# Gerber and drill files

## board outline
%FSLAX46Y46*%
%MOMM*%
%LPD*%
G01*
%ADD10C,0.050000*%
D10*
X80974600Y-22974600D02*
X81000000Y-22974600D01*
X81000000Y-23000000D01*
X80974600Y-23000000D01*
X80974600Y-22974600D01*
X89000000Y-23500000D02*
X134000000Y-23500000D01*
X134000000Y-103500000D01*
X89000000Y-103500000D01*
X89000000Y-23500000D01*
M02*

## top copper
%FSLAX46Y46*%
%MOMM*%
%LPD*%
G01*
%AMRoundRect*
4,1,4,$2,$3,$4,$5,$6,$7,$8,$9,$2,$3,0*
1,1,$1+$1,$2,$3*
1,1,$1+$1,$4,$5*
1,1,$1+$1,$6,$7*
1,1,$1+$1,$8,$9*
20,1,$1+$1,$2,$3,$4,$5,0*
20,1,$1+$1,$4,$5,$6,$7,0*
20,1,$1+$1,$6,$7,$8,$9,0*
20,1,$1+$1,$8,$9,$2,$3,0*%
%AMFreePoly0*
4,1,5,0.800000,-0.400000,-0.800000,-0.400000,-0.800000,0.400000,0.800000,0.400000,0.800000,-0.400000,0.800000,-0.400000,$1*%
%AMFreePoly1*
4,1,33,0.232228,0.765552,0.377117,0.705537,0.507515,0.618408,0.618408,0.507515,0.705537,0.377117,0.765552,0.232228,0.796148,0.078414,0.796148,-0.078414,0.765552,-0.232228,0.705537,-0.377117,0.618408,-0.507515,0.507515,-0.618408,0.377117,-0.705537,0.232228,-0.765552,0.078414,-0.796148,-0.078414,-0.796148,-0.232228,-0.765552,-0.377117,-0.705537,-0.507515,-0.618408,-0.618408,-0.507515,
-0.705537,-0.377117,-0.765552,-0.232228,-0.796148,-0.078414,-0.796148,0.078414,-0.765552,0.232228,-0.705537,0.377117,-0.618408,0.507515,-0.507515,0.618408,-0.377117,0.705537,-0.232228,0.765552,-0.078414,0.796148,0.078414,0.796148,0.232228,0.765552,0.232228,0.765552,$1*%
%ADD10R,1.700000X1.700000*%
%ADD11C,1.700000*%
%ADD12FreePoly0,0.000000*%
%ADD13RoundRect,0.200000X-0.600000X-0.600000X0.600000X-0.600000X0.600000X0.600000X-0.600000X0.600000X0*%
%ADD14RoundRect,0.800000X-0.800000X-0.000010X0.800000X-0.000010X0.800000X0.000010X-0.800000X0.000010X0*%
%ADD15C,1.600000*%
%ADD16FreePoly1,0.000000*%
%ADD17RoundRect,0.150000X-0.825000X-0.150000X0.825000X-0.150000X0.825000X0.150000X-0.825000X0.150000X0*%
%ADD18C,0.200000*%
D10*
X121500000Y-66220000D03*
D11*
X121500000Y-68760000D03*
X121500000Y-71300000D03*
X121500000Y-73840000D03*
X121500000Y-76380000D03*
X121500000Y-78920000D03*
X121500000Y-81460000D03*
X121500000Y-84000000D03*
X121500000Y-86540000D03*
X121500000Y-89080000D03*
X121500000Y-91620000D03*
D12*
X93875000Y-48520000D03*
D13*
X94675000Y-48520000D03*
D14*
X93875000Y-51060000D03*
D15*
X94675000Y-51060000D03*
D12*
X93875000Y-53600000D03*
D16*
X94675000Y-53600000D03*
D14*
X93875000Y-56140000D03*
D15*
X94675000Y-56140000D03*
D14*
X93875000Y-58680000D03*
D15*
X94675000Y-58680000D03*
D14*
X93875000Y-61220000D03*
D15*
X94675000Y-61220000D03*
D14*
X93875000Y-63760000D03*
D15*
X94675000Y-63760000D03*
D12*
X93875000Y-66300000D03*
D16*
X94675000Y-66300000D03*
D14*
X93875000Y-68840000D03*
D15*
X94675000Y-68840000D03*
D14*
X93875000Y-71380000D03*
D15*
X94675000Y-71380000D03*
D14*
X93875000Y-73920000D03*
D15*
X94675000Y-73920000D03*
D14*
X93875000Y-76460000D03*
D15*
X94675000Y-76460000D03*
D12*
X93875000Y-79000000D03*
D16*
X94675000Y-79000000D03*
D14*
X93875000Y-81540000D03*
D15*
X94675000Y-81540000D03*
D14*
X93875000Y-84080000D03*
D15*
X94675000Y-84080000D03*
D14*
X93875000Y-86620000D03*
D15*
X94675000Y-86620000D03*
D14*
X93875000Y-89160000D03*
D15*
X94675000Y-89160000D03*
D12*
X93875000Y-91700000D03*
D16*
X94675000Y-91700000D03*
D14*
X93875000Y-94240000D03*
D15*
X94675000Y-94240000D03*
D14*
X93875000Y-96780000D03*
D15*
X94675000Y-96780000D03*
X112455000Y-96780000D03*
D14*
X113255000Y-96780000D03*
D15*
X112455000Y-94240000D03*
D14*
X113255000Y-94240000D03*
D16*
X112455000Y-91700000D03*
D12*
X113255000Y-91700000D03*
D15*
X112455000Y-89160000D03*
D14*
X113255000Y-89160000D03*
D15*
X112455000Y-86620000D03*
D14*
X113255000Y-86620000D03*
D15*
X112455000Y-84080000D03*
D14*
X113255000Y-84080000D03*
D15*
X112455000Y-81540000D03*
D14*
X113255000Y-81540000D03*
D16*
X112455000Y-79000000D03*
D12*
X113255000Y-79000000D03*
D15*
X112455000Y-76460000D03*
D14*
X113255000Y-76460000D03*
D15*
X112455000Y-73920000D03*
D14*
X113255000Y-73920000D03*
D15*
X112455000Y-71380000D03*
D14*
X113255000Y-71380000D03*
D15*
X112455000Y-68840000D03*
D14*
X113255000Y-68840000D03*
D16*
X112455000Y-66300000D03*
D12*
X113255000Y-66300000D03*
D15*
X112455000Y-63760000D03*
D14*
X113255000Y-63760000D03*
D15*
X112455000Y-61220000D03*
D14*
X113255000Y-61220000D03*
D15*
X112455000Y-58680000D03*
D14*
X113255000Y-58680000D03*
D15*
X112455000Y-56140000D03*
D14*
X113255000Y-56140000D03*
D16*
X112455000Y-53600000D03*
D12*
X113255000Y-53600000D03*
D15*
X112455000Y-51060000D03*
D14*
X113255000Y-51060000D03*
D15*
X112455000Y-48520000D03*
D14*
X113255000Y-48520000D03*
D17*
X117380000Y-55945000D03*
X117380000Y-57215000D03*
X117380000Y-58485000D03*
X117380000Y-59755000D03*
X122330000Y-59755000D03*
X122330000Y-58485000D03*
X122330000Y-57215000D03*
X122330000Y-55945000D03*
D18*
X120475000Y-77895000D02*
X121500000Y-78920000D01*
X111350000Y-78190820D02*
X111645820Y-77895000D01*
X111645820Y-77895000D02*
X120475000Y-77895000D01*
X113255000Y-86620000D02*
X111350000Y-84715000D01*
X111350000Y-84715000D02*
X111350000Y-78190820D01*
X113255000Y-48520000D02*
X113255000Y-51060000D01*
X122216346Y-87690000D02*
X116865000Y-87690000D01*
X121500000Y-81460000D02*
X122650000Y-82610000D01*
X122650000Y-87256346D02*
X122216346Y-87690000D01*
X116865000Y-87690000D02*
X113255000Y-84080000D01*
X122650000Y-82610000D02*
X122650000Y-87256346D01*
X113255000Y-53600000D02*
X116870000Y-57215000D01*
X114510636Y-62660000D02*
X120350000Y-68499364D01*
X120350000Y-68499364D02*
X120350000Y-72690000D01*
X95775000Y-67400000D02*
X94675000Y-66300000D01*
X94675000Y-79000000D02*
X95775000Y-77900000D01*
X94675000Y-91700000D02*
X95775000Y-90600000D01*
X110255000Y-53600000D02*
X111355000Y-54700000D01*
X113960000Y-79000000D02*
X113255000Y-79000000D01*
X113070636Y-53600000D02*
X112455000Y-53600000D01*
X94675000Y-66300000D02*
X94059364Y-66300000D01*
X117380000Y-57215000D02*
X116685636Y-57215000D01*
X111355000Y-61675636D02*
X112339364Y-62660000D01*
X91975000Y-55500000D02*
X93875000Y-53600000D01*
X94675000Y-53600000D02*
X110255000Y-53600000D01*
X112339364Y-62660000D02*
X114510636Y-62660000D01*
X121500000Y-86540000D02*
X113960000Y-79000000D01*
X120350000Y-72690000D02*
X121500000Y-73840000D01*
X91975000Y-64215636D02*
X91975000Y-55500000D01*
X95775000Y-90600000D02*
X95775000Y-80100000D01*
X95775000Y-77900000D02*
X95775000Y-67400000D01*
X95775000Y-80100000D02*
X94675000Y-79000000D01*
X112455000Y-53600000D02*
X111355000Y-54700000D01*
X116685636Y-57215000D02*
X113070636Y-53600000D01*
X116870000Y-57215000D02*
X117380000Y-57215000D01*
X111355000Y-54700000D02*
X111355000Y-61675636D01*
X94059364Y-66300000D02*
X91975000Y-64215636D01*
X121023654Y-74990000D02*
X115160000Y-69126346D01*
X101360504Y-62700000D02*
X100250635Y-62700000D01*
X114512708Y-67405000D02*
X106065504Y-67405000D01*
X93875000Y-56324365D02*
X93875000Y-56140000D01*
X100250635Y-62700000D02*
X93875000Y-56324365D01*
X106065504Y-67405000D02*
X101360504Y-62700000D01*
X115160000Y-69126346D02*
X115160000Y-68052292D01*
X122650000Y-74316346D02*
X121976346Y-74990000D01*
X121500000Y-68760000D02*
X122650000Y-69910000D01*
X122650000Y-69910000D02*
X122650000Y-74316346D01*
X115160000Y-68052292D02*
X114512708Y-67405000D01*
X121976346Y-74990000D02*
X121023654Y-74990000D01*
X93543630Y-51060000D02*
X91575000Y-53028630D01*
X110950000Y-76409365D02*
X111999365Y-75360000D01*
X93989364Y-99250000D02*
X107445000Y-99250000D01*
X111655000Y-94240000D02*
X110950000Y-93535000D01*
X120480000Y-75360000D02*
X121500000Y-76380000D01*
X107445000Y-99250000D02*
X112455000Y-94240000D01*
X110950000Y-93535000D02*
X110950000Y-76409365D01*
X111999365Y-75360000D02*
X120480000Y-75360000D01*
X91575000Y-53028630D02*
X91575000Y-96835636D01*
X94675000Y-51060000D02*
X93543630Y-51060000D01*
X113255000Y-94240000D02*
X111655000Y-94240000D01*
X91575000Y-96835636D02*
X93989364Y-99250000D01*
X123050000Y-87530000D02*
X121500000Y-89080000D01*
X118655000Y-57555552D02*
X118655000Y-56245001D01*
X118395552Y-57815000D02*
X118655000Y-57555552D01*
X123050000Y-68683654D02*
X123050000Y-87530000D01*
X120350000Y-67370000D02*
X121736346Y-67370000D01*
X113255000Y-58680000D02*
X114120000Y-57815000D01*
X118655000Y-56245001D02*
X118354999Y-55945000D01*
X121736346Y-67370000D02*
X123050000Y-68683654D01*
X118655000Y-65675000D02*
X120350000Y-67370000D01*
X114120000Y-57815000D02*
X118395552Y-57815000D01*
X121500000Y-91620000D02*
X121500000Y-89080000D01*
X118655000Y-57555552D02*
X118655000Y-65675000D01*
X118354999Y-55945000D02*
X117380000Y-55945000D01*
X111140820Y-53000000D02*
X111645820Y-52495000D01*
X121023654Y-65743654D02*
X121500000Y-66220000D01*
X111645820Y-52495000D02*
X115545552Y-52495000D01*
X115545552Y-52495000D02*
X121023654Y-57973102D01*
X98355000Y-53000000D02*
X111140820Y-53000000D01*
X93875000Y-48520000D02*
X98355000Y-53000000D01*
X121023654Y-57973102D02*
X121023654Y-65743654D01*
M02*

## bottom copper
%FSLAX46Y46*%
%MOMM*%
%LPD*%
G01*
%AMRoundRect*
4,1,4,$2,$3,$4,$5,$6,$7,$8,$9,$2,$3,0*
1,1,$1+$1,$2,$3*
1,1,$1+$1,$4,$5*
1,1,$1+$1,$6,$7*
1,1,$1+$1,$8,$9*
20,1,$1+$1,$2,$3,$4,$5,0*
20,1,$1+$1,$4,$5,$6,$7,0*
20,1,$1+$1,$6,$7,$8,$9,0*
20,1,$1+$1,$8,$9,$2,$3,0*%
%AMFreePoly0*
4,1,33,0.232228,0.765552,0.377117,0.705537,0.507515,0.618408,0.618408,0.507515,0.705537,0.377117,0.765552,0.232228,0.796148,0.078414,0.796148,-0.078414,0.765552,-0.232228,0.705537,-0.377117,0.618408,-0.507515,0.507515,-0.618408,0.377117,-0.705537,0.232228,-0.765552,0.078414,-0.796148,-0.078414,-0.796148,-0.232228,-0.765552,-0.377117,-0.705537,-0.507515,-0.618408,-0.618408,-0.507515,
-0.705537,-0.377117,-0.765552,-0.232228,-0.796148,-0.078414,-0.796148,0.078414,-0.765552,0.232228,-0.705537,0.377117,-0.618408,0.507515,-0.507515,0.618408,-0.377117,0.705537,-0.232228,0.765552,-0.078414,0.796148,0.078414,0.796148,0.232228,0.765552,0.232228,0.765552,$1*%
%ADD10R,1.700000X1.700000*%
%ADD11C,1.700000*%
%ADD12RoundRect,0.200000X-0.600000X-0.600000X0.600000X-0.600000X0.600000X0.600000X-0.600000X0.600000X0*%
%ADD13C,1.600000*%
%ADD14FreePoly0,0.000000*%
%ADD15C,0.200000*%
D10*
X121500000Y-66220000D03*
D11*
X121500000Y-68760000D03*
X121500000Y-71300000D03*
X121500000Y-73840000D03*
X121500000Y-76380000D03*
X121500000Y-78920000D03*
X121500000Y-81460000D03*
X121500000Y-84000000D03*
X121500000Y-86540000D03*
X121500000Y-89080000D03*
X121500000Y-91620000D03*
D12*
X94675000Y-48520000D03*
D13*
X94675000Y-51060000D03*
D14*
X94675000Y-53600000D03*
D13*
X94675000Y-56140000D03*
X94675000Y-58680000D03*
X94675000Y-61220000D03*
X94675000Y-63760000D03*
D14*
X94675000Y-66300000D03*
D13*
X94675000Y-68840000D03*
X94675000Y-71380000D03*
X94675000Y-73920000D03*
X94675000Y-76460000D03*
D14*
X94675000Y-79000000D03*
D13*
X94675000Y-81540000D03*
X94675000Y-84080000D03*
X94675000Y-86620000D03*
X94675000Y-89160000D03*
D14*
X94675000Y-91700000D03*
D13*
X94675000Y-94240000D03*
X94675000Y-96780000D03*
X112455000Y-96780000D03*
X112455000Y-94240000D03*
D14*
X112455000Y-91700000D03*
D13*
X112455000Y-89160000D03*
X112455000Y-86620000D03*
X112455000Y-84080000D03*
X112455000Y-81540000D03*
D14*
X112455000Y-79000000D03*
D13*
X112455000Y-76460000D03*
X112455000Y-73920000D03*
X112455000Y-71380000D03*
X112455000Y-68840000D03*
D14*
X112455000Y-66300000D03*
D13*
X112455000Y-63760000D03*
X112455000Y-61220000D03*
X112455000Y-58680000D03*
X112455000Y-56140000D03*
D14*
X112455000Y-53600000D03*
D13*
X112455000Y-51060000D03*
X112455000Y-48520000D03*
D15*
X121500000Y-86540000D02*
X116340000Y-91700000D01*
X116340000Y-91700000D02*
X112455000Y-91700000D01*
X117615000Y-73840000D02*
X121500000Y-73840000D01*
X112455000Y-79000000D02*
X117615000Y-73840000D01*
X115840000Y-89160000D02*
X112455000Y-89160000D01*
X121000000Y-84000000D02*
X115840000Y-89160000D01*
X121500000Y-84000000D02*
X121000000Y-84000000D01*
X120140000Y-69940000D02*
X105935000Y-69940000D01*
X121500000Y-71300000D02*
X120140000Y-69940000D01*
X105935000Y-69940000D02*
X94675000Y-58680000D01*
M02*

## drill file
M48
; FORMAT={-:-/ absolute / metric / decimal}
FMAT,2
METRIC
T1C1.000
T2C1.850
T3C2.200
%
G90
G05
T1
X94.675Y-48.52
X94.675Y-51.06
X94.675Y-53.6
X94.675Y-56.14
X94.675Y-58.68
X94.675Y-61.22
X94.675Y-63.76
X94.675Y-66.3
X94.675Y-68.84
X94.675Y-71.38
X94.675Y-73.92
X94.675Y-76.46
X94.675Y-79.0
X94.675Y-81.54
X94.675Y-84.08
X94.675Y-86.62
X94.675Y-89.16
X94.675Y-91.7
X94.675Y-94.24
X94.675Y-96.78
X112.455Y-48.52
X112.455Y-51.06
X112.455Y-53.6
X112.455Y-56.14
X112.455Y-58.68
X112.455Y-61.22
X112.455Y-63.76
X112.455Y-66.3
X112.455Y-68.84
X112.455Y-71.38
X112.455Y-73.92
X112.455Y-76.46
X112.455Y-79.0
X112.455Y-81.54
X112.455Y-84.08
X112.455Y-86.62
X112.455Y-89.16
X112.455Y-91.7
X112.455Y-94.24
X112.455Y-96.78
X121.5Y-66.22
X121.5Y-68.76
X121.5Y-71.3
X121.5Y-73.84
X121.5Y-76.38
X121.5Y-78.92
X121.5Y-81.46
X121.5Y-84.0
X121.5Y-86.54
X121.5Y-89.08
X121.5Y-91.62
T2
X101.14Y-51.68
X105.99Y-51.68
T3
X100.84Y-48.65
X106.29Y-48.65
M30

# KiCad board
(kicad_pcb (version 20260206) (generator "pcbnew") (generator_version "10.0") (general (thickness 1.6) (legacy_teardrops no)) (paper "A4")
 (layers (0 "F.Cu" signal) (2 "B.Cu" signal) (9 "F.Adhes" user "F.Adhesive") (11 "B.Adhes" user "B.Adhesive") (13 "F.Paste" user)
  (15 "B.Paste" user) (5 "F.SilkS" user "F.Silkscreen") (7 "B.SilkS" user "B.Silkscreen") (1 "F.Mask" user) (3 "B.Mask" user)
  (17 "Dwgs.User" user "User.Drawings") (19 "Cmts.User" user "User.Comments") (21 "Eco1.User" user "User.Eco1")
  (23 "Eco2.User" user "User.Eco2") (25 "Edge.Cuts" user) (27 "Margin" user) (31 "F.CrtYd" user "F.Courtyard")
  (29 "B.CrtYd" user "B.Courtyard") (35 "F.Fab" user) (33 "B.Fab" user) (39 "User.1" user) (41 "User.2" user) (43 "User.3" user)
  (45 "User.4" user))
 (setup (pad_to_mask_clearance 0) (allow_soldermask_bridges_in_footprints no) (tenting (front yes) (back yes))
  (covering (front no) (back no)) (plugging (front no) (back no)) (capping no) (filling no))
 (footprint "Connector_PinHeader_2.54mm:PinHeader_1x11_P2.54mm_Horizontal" (layer "F.Cu") (at 121.5 66.22)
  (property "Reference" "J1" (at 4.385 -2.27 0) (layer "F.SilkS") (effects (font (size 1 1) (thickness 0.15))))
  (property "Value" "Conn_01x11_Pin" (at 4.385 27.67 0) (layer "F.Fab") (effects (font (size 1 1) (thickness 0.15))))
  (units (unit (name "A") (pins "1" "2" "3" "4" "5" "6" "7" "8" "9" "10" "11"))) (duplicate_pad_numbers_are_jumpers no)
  (pad "1" thru_hole rect (at 0 0) (size 1.7 1.7) (drill 1) (layers "*.Cu" "*.Mask") (remove_unused_layers no) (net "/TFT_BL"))
  (pad "2" thru_hole circle (at 0 2.54) (size 1.7 1.7) (drill 1) (layers "*.Cu" "*.Mask") (remove_unused_layers no) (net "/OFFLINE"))
  (pad "3" thru_hole circle (at 0 5.08) (size 1.7 1.7) (drill 1) (layers "*.Cu" "*.Mask") (remove_unused_layers no) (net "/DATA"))
  (pad "4" thru_hole circle (at 0 7.62) (size 1.7 1.7) (drill 1) (layers "*.Cu" "*.Mask") (remove_unused_layers no) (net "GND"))
  (pad "5" thru_hole circle (at 0 10.16) (size 1.7 1.7) (drill 1) (layers "*.Cu" "*.Mask") (remove_unused_layers no) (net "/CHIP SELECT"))
  (pad "6" thru_hole circle (at 0 12.7) (size 1.7 1.7) (drill 1) (layers "*.Cu" "*.Mask") (remove_unused_layers no) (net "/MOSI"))
  (pad "7" thru_hole circle (at 0 15.24) (size 1.7 1.7) (drill 1) (layers "*.Cu" "*.Mask") (remove_unused_layers no) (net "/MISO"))
  (pad "8" thru_hole circle (at 0 17.78) (size 1.7 1.7) (drill 1) (layers "*.Cu" "*.Mask") (remove_unused_layers no) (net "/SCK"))
  (pad "9" thru_hole circle (at 0 20.32) (size 1.7 1.7) (drill 1) (layers "*.Cu" "*.Mask") (remove_unused_layers no) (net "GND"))
  (pad "10" thru_hole circle (at 0 22.86) (size 1.7 1.7) (drill 1) (layers "*.Cu" "*.Mask") (remove_unused_layers no) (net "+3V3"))
  (pad "11" thru_hole circle (at 0 25.4) (size 1.7 1.7) (drill 1) (layers "*.Cu" "*.Mask") (remove_unused_layers no) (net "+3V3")))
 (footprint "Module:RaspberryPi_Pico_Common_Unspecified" (layer "F.Cu") (at 103.565 72.65)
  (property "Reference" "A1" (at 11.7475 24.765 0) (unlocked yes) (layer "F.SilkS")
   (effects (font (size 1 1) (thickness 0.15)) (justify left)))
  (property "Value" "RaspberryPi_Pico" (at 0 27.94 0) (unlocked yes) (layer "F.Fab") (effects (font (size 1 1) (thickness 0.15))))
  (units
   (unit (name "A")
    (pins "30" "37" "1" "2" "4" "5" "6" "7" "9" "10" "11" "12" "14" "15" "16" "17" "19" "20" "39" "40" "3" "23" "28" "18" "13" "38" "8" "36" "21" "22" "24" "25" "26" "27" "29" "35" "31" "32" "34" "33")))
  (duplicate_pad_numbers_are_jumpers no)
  (pad "" np_thru_hole circle (at -2.725 -24) (size 2.2 2.2) (drill 2.2) (layers "*.Mask"))
  (pad "" np_thru_hole circle (at -2.425 -20.97) (size 1.85 1.85) (drill 1.85) (layers "*.Mask"))
  (pad "" np_thru_hole circle (at 2.425 -20.97) (size 1.85 1.85) (drill 1.85) (layers "*.Mask"))
  (pad "" np_thru_hole circle (at 2.725 -24) (size 2.2 2.2) (drill 2.2) (layers "*.Mask"))
  (pad "1" smd custom (at -9.69 -24.13) (size 1.6 0.8) (layers "F.Cu" "F.Mask") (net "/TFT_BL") (options (clearance outline) (anchor rect))
   (primitives))
  (pad "1" thru_hole roundrect (at -8.89 -24.13) (size 1.6 1.6) (drill 1) (layers "*.Cu" "*.Mask") (remove_unused_layers no)
   (roundrect_rratio 0.125) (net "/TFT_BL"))
  (pad "2" smd roundrect (at -9.69 -21.59) (size 3.2 1.6) (layers "F.Cu" "F.Mask") (roundrect_rratio 0.5) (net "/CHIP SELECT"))
  (pad "2" thru_hole circle (at -8.89 -21.59) (size 1.6 1.6) (drill 1) (layers "*.Cu" "*.Mask") (remove_unused_layers no)
   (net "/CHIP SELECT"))
  (pad "3" smd custom (at -9.69 -19.05) (size 1.6 0.8) (layers "F.Cu" "F.Mask") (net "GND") (options (clearance outline) (anchor rect))
   (primitives))
  (pad "3" thru_hole custom (at -8.89 -19.05) (size 1.6 1.6) (drill 1) (layers "*.Cu" "*.Mask") (remove_unused_layers no) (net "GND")
   (options (clearance outline) (anchor circle)) (primitives))
  (pad "4" smd roundrect (at -9.69 -16.51) (size 3.2 1.6) (layers "F.Cu" "F.Mask") (roundrect_rratio 0.5) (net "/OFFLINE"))
  (pad "4" thru_hole circle (at -8.89 -16.51) (size 1.6 1.6) (drill 1) (layers "*.Cu" "*.Mask") (remove_unused_layers no) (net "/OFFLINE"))
  (pad "5" smd roundrect (at -9.69 -13.97) (size 3.2 1.6) (layers "F.Cu" "F.Mask") (roundrect_rratio 0.5) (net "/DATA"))
  (pad "5" thru_hole circle (at -8.89 -13.97) (size 1.6 1.6) (drill 1) (layers "*.Cu" "*.Mask") (remove_unused_layers no) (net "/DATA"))
  (pad "6" smd roundrect (at -9.69 -11.43) (size 3.2 1.6) (layers "F.Cu" "F.Mask") (roundrect_rratio 0.5)
   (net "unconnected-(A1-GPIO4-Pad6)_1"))
  (pad "6" thru_hole circle (at -8.89 -11.43) (size 1.6 1.6) (drill 1) (layers "*.Cu" "*.Mask") (remove_unused_layers no)
   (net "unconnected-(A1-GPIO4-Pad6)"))
  (pad "7" smd roundrect (at -9.69 -8.89) (size 3.2 1.6) (layers "F.Cu" "F.Mask") (roundrect_rratio 0.5)
   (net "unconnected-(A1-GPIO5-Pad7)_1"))
  (pad "7" thru_hole circle (at -8.89 -8.89) (size 1.6 1.6) (drill 1) (layers "*.Cu" "*.Mask") (remove_unused_layers no)
   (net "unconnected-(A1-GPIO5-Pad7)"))
  (pad "8" smd custom (at -9.69 -6.35) (size 1.6 0.8) (layers "F.Cu" "F.Mask") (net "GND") (options (clearance outline) (anchor rect))
   (primitives))
  (pad "8" thru_hole custom (at -8.89 -6.35) (size 1.6 1.6) (drill 1) (layers "*.Cu" "*.Mask") (remove_unused_layers no) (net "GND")
   (options (clearance outline) (anchor circle)) (primitives))
  (pad "9" smd roundrect (at -9.69 -3.81) (size 3.2 1.6) (layers "F.Cu" "F.Mask") (roundrect_rratio 0.5) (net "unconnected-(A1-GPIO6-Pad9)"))
  (pad "9" thru_hole circle (at -8.89 -3.81) (size 1.6 1.6) (drill 1) (layers "*.Cu" "*.Mask") (remove_unused_layers no)
   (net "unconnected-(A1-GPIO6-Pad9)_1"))
  (pad "10" smd roundrect (at -9.69 -1.27) (size 3.2 1.6) (layers "F.Cu" "F.Mask") (roundrect_rratio 0.5)
   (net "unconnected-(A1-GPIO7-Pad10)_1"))
  (pad "10" thru_hole circle (at -8.89 -1.27) (size 1.6 1.6) (drill 1) (layers "*.Cu" "*.Mask") (remove_unused_layers no)
   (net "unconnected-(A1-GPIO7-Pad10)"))
  (pad "11" smd roundrect (at -9.69 1.27) (size 3.2 1.6) (layers "F.Cu" "F.Mask") (roundrect_rratio 0.5)
   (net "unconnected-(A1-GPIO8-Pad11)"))
  (pad "11" thru_hole circle (at -8.89 1.27) (size 1.6 1.6) (drill 1) (layers "*.Cu" "*.Mask") (remove_unused_layers no)
   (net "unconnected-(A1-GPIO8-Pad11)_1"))
  (pad "12" smd roundrect (at -9.69 3.81) (size 3.2 1.6) (layers "F.Cu" "F.Mask") (roundrect_rratio 0.5)
   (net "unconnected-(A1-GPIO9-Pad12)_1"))
  (pad "12" thru_hole circle (at -8.89 3.81) (size 1.6 1.6) (drill 1) (layers "*.Cu" "*.Mask") (remove_unused_layers no)
   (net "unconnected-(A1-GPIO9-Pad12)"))
  (pad "13" smd custom (at -9.69 6.35) (size 1.6 0.8) (layers "F.Cu" "F.Mask") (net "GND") (options (clearance outline) (anchor rect))
   (primitives))
  (pad "13" thru_hole custom (at -8.89 6.35) (size 1.6 1.6) (drill 1) (layers "*.Cu" "*.Mask") (remove_unused_layers no) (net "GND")
   (options (clearance outline) (anchor circle)) (primitives))
  (pad "14" smd roundrect (at -9.69 8.89) (size 3.2 1.6) (layers "F.Cu" "F.Mask") (roundrect_rratio 0.5)
   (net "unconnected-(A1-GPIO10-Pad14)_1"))
  (pad "14" thru_hole circle (at -8.89 8.89) (size 1.6 1.6) (drill 1) (layers "*.Cu" "*.Mask") (remove_unused_layers no)
   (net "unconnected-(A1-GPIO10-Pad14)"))
  (pad "15" smd roundrect (at -9.69 11.43) (size 3.2 1.6) (layers "F.Cu" "F.Mask") (roundrect_rratio 0.5)
   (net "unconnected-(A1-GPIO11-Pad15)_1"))
  (pad "15" thru_hole circle (at -8.89 11.43) (size 1.6 1.6) (drill 1) (layers "*.Cu" "*.Mask") (remove_unused_layers no)
   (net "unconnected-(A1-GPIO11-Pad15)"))
  (pad "16" smd roundrect (at -9.69 13.97) (size 3.2 1.6) (layers "F.Cu" "F.Mask") (roundrect_rratio 0.5)
   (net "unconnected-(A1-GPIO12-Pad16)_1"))
  (pad "16" thru_hole circle (at -8.89 13.97) (size 1.6 1.6) (drill 1) (layers "*.Cu" "*.Mask") (remove_unused_layers no)
   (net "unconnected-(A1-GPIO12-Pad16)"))
  (pad "17" smd roundrect (at -9.69 16.51) (size 3.2 1.6) (layers "F.Cu" "F.Mask") (roundrect_rratio 0.5)
   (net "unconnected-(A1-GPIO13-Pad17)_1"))
  (pad "17" thru_hole circle (at -8.89 16.51) (size 1.6 1.6) (drill 1) (layers "*.Cu" "*.Mask") (remove_unused_layers no)
   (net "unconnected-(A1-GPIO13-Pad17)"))
  (pad "18" smd custom (at -9.69 19.05) (size 1.6 0.8) (layers "F.Cu" "F.Mask") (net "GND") (options (clearance outline) (anchor rect))
   (primitives))
  (pad "18" thru_hole custom (at -8.89 19.05) (size 1.6 1.6) (drill 1) (layers "*.Cu" "*.Mask") (remove_unused_layers no) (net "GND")
   (options (clearance outline) (anchor circle)) (primitives))
  (pad "19" smd roundrect (at -9.69 21.59) (size 3.2 1.6) (layers "F.Cu" "F.Mask") (roundrect_rratio 0.5)
   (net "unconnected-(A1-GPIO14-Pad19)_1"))
  (pad "19" thru_hole circle (at -8.89 21.59) (size 1.6 1.6) (drill 1) (layers "*.Cu" "*.Mask") (remove_unused_layers no)
   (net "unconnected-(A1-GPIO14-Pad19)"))
  (pad "20" smd roundrect (at -9.69 24.13) (size 3.2 1.6) (layers "F.Cu" "F.Mask") (roundrect_rratio 0.5)
   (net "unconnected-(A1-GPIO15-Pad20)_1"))
  (pad "20" thru_hole circle (at -8.89 24.13) (size 1.6 1.6) (drill 1) (layers "*.Cu" "*.Mask") (remove_unused_layers no)
   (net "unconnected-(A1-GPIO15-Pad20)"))
  (pad "21" thru_hole circle (at 8.89 24.13) (size 1.6 1.6) (drill 1) (layers "*.Cu" "*.Mask") (remove_unused_layers no)
   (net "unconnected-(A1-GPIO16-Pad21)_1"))
  (pad "21" smd roundrect (at 9.69 24.13) (size 3.2 1.6) (layers "F.Cu" "F.Mask") (roundrect_rratio 0.5)
   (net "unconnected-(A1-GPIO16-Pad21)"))
  (pad "22" thru_hole circle (at 8.89 21.59) (size 1.6 1.6) (drill 1) (layers "*.Cu" "*.Mask") (remove_unused_layers no)
   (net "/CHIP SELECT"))
  (pad "22" smd roundrect (at 9.69 21.59) (size 3.2 1.6) (layers "F.Cu" "F.Mask") (roundrect_rratio 0.5) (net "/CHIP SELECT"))
  (pad "23" thru_hole custom (at 8.89 19.05) (size 1.6 1.6) (drill 1) (layers "*.Cu" "*.Mask") (remove_unused_layers no) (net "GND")
   (options (clearance outline) (anchor circle)) (primitives))
  (pad "23" smd custom (at 9.69 19.05) (size 1.6 0.8) (layers "F.Cu" "F.Mask") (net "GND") (options (clearance outline) (anchor rect))
   (primitives))
  (pad "24" thru_hole circle (at 8.89 16.51) (size 1.6 1.6) (drill 1) (layers "*.Cu" "*.Mask") (remove_unused_layers no) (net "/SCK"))
  (pad "24" smd roundrect (at 9.69 16.51) (size 3.2 1.6) (layers "F.Cu" "F.Mask") (roundrect_rratio 0.5) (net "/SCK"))
  (pad "25" thru_hole circle (at 8.89 13.97) (size 1.6 1.6) (drill 1) (layers "*.Cu" "*.Mask") (remove_unused_layers no) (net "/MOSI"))
  (pad "25" smd roundrect (at 9.69 13.97) (size 3.2 1.6) (layers "F.Cu" "F.Mask") (roundrect_rratio 0.5) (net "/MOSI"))
  (pad "26" thru_hole circle (at 8.89 11.43) (size 1.6 1.6) (drill 1) (layers "*.Cu" "*.Mask") (remove_unused_layers no) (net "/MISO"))
  (pad "26" smd roundrect (at 9.69 11.43) (size 3.2 1.6) (layers "F.Cu" "F.Mask") (roundrect_rratio 0.5) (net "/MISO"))
  (pad "27" thru_hole circle (at 8.89 8.89) (size 1.6 1.6) (drill 1) (layers "*.Cu" "*.Mask") (remove_unused_layers no)
   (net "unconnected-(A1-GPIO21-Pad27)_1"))
  (pad "27" smd roundrect (at 9.69 8.89) (size 3.2 1.6) (layers "F.Cu" "F.Mask") (roundrect_rratio 0.5)
   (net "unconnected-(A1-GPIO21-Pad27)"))
  (pad "28" thru_hole custom (at 8.89 6.35) (size 1.6 1.6) (drill 1) (layers "*.Cu" "*.Mask") (remove_unused_layers no) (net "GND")
   (options (clearance outline) (anchor circle)) (primitives))
  (pad "28" smd custom (at 9.69 6.35) (size 1.6 0.8) (layers "F.Cu" "F.Mask") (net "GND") (options (clearance outline) (anchor rect))
   (primitives))
  (pad "29" thru_hole circle (at 8.89 3.81) (size 1.6 1.6) (drill 1) (layers "*.Cu" "*.Mask") (remove_unused_layers no)
   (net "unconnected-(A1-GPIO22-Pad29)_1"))
  (pad "29" smd roundrect (at 9.69 3.81) (size 3.2 1.6) (layers "F.Cu" "F.Mask") (roundrect_rratio 0.5)
   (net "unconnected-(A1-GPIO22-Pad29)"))
  (pad "30" thru_hole circle (at 8.89 1.27) (size 1.6 1.6) (drill 1) (layers "*.Cu" "*.Mask") (remove_unused_layers no)
   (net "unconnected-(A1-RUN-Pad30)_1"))
  (pad "30" smd roundrect (at 9.69 1.27) (size 3.2 1.6) (layers "F.Cu" "F.Mask") (roundrect_rratio 0.5) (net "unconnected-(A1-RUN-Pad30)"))
  (pad "31" thru_hole circle (at 8.89 -1.27) (size 1.6 1.6) (drill 1) (layers "*.Cu" "*.Mask") (remove_unused_layers no)
   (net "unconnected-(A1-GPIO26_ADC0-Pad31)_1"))
  (pad "31" smd roundrect (at 9.69 -1.27) (size 3.2 1.6) (layers "F.Cu" "F.Mask") (roundrect_rratio 0.5)
   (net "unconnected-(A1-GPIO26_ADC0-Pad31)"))
  (pad "32" thru_hole circle (at 8.89 -3.81) (size 1.6 1.6) (drill 1) (layers "*.Cu" "*.Mask") (remove_unused_layers no)
   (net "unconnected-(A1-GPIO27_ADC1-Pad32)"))
  (pad "32" smd roundrect (at 9.69 -3.81) (size 3.2 1.6) (layers "F.Cu" "F.Mask") (roundrect_rratio 0.5)
   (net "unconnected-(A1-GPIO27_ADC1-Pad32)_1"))
  (pad "33" thru_hole custom (at 8.89 -6.35) (size 1.6 1.6) (drill 1) (layers "*.Cu" "*.Mask") (remove_unused_layers no) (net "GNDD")
   (options (clearance outline) (anchor circle)) (primitives))
  (pad "33" smd custom (at 9.69 -6.35) (size 1.6 0.8) (layers "F.Cu" "F.Mask") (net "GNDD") (options (clearance outline) (anchor rect))
   (primitives))
  (pad "34" thru_hole circle (at 8.89 -8.89) (size 1.6 1.6) (drill 1) (layers "*.Cu" "*.Mask") (remove_unused_layers no)
   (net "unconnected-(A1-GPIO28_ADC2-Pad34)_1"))
  (pad "34" smd roundrect (at 9.69 -8.89) (size 3.2 1.6) (layers "F.Cu" "F.Mask") (roundrect_rratio 0.5)
   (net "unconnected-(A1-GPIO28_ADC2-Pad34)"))
  (pad "35" thru_hole circle (at 8.89 -11.43) (size 1.6 1.6) (drill 1) (layers "*.Cu" "*.Mask") (remove_unused_layers no)
   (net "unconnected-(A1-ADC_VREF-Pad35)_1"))
  (pad "35" smd roundrect (at 9.69 -11.43) (size 3.2 1.6) (layers "F.Cu" "F.Mask") (roundrect_rratio 0.5)
   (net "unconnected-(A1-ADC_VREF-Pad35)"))
  (pad "36" thru_hole circle (at 8.89 -13.97) (size 1.6 1.6) (drill 1) (layers "*.Cu" "*.Mask") (remove_unused_layers no) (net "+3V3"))
  (pad "36" smd roundrect (at 9.69 -13.97) (size 3.2 1.6) (layers "F.Cu" "F.Mask") (roundrect_rratio 0.5) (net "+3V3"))
  (pad "37" thru_hole circle (at 8.89 -16.51) (size 1.6 1.6) (drill 1) (layers "*.Cu" "*.Mask") (remove_unused_layers no)
   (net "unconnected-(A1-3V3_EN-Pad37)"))
  (pad "37" smd roundrect (at 9.69 -16.51) (size 3.2 1.6) (layers "F.Cu" "F.Mask") (roundrect_rratio 0.5)
   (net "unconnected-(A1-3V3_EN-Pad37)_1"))
  (pad "38" thru_hole custom (at 8.89 -19.05) (size 1.6 1.6) (drill 1) (layers "*.Cu" "*.Mask") (remove_unused_layers no) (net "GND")
   (options (clearance outline) (anchor circle)) (primitives))
  (pad "38" smd custom (at 9.69 -19.05) (size 1.6 0.8) (layers "F.Cu" "F.Mask") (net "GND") (options (clearance outline) (anchor rect))
   (primitives))
  (pad "39" thru_hole circle (at 8.89 -21.59) (size 1.6 1.6) (drill 1) (layers "*.Cu" "*.Mask") (remove_unused_layers no) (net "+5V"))
  (pad "39" smd roundrect (at 9.69 -21.59) (size 3.2 1.6) (layers "F.Cu" "F.Mask") (roundrect_rratio 0.5) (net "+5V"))
  (pad "40" thru_hole circle (at 8.89 -24.13) (size 1.6 1.6) (drill 1) (layers "*.Cu" "*.Mask") (remove_unused_layers no) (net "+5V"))
  (pad "40" smd roundrect (at 9.69 -24.13) (size 3.2 1.6) (layers "F.Cu" "F.Mask") (roundrect_rratio 0.5) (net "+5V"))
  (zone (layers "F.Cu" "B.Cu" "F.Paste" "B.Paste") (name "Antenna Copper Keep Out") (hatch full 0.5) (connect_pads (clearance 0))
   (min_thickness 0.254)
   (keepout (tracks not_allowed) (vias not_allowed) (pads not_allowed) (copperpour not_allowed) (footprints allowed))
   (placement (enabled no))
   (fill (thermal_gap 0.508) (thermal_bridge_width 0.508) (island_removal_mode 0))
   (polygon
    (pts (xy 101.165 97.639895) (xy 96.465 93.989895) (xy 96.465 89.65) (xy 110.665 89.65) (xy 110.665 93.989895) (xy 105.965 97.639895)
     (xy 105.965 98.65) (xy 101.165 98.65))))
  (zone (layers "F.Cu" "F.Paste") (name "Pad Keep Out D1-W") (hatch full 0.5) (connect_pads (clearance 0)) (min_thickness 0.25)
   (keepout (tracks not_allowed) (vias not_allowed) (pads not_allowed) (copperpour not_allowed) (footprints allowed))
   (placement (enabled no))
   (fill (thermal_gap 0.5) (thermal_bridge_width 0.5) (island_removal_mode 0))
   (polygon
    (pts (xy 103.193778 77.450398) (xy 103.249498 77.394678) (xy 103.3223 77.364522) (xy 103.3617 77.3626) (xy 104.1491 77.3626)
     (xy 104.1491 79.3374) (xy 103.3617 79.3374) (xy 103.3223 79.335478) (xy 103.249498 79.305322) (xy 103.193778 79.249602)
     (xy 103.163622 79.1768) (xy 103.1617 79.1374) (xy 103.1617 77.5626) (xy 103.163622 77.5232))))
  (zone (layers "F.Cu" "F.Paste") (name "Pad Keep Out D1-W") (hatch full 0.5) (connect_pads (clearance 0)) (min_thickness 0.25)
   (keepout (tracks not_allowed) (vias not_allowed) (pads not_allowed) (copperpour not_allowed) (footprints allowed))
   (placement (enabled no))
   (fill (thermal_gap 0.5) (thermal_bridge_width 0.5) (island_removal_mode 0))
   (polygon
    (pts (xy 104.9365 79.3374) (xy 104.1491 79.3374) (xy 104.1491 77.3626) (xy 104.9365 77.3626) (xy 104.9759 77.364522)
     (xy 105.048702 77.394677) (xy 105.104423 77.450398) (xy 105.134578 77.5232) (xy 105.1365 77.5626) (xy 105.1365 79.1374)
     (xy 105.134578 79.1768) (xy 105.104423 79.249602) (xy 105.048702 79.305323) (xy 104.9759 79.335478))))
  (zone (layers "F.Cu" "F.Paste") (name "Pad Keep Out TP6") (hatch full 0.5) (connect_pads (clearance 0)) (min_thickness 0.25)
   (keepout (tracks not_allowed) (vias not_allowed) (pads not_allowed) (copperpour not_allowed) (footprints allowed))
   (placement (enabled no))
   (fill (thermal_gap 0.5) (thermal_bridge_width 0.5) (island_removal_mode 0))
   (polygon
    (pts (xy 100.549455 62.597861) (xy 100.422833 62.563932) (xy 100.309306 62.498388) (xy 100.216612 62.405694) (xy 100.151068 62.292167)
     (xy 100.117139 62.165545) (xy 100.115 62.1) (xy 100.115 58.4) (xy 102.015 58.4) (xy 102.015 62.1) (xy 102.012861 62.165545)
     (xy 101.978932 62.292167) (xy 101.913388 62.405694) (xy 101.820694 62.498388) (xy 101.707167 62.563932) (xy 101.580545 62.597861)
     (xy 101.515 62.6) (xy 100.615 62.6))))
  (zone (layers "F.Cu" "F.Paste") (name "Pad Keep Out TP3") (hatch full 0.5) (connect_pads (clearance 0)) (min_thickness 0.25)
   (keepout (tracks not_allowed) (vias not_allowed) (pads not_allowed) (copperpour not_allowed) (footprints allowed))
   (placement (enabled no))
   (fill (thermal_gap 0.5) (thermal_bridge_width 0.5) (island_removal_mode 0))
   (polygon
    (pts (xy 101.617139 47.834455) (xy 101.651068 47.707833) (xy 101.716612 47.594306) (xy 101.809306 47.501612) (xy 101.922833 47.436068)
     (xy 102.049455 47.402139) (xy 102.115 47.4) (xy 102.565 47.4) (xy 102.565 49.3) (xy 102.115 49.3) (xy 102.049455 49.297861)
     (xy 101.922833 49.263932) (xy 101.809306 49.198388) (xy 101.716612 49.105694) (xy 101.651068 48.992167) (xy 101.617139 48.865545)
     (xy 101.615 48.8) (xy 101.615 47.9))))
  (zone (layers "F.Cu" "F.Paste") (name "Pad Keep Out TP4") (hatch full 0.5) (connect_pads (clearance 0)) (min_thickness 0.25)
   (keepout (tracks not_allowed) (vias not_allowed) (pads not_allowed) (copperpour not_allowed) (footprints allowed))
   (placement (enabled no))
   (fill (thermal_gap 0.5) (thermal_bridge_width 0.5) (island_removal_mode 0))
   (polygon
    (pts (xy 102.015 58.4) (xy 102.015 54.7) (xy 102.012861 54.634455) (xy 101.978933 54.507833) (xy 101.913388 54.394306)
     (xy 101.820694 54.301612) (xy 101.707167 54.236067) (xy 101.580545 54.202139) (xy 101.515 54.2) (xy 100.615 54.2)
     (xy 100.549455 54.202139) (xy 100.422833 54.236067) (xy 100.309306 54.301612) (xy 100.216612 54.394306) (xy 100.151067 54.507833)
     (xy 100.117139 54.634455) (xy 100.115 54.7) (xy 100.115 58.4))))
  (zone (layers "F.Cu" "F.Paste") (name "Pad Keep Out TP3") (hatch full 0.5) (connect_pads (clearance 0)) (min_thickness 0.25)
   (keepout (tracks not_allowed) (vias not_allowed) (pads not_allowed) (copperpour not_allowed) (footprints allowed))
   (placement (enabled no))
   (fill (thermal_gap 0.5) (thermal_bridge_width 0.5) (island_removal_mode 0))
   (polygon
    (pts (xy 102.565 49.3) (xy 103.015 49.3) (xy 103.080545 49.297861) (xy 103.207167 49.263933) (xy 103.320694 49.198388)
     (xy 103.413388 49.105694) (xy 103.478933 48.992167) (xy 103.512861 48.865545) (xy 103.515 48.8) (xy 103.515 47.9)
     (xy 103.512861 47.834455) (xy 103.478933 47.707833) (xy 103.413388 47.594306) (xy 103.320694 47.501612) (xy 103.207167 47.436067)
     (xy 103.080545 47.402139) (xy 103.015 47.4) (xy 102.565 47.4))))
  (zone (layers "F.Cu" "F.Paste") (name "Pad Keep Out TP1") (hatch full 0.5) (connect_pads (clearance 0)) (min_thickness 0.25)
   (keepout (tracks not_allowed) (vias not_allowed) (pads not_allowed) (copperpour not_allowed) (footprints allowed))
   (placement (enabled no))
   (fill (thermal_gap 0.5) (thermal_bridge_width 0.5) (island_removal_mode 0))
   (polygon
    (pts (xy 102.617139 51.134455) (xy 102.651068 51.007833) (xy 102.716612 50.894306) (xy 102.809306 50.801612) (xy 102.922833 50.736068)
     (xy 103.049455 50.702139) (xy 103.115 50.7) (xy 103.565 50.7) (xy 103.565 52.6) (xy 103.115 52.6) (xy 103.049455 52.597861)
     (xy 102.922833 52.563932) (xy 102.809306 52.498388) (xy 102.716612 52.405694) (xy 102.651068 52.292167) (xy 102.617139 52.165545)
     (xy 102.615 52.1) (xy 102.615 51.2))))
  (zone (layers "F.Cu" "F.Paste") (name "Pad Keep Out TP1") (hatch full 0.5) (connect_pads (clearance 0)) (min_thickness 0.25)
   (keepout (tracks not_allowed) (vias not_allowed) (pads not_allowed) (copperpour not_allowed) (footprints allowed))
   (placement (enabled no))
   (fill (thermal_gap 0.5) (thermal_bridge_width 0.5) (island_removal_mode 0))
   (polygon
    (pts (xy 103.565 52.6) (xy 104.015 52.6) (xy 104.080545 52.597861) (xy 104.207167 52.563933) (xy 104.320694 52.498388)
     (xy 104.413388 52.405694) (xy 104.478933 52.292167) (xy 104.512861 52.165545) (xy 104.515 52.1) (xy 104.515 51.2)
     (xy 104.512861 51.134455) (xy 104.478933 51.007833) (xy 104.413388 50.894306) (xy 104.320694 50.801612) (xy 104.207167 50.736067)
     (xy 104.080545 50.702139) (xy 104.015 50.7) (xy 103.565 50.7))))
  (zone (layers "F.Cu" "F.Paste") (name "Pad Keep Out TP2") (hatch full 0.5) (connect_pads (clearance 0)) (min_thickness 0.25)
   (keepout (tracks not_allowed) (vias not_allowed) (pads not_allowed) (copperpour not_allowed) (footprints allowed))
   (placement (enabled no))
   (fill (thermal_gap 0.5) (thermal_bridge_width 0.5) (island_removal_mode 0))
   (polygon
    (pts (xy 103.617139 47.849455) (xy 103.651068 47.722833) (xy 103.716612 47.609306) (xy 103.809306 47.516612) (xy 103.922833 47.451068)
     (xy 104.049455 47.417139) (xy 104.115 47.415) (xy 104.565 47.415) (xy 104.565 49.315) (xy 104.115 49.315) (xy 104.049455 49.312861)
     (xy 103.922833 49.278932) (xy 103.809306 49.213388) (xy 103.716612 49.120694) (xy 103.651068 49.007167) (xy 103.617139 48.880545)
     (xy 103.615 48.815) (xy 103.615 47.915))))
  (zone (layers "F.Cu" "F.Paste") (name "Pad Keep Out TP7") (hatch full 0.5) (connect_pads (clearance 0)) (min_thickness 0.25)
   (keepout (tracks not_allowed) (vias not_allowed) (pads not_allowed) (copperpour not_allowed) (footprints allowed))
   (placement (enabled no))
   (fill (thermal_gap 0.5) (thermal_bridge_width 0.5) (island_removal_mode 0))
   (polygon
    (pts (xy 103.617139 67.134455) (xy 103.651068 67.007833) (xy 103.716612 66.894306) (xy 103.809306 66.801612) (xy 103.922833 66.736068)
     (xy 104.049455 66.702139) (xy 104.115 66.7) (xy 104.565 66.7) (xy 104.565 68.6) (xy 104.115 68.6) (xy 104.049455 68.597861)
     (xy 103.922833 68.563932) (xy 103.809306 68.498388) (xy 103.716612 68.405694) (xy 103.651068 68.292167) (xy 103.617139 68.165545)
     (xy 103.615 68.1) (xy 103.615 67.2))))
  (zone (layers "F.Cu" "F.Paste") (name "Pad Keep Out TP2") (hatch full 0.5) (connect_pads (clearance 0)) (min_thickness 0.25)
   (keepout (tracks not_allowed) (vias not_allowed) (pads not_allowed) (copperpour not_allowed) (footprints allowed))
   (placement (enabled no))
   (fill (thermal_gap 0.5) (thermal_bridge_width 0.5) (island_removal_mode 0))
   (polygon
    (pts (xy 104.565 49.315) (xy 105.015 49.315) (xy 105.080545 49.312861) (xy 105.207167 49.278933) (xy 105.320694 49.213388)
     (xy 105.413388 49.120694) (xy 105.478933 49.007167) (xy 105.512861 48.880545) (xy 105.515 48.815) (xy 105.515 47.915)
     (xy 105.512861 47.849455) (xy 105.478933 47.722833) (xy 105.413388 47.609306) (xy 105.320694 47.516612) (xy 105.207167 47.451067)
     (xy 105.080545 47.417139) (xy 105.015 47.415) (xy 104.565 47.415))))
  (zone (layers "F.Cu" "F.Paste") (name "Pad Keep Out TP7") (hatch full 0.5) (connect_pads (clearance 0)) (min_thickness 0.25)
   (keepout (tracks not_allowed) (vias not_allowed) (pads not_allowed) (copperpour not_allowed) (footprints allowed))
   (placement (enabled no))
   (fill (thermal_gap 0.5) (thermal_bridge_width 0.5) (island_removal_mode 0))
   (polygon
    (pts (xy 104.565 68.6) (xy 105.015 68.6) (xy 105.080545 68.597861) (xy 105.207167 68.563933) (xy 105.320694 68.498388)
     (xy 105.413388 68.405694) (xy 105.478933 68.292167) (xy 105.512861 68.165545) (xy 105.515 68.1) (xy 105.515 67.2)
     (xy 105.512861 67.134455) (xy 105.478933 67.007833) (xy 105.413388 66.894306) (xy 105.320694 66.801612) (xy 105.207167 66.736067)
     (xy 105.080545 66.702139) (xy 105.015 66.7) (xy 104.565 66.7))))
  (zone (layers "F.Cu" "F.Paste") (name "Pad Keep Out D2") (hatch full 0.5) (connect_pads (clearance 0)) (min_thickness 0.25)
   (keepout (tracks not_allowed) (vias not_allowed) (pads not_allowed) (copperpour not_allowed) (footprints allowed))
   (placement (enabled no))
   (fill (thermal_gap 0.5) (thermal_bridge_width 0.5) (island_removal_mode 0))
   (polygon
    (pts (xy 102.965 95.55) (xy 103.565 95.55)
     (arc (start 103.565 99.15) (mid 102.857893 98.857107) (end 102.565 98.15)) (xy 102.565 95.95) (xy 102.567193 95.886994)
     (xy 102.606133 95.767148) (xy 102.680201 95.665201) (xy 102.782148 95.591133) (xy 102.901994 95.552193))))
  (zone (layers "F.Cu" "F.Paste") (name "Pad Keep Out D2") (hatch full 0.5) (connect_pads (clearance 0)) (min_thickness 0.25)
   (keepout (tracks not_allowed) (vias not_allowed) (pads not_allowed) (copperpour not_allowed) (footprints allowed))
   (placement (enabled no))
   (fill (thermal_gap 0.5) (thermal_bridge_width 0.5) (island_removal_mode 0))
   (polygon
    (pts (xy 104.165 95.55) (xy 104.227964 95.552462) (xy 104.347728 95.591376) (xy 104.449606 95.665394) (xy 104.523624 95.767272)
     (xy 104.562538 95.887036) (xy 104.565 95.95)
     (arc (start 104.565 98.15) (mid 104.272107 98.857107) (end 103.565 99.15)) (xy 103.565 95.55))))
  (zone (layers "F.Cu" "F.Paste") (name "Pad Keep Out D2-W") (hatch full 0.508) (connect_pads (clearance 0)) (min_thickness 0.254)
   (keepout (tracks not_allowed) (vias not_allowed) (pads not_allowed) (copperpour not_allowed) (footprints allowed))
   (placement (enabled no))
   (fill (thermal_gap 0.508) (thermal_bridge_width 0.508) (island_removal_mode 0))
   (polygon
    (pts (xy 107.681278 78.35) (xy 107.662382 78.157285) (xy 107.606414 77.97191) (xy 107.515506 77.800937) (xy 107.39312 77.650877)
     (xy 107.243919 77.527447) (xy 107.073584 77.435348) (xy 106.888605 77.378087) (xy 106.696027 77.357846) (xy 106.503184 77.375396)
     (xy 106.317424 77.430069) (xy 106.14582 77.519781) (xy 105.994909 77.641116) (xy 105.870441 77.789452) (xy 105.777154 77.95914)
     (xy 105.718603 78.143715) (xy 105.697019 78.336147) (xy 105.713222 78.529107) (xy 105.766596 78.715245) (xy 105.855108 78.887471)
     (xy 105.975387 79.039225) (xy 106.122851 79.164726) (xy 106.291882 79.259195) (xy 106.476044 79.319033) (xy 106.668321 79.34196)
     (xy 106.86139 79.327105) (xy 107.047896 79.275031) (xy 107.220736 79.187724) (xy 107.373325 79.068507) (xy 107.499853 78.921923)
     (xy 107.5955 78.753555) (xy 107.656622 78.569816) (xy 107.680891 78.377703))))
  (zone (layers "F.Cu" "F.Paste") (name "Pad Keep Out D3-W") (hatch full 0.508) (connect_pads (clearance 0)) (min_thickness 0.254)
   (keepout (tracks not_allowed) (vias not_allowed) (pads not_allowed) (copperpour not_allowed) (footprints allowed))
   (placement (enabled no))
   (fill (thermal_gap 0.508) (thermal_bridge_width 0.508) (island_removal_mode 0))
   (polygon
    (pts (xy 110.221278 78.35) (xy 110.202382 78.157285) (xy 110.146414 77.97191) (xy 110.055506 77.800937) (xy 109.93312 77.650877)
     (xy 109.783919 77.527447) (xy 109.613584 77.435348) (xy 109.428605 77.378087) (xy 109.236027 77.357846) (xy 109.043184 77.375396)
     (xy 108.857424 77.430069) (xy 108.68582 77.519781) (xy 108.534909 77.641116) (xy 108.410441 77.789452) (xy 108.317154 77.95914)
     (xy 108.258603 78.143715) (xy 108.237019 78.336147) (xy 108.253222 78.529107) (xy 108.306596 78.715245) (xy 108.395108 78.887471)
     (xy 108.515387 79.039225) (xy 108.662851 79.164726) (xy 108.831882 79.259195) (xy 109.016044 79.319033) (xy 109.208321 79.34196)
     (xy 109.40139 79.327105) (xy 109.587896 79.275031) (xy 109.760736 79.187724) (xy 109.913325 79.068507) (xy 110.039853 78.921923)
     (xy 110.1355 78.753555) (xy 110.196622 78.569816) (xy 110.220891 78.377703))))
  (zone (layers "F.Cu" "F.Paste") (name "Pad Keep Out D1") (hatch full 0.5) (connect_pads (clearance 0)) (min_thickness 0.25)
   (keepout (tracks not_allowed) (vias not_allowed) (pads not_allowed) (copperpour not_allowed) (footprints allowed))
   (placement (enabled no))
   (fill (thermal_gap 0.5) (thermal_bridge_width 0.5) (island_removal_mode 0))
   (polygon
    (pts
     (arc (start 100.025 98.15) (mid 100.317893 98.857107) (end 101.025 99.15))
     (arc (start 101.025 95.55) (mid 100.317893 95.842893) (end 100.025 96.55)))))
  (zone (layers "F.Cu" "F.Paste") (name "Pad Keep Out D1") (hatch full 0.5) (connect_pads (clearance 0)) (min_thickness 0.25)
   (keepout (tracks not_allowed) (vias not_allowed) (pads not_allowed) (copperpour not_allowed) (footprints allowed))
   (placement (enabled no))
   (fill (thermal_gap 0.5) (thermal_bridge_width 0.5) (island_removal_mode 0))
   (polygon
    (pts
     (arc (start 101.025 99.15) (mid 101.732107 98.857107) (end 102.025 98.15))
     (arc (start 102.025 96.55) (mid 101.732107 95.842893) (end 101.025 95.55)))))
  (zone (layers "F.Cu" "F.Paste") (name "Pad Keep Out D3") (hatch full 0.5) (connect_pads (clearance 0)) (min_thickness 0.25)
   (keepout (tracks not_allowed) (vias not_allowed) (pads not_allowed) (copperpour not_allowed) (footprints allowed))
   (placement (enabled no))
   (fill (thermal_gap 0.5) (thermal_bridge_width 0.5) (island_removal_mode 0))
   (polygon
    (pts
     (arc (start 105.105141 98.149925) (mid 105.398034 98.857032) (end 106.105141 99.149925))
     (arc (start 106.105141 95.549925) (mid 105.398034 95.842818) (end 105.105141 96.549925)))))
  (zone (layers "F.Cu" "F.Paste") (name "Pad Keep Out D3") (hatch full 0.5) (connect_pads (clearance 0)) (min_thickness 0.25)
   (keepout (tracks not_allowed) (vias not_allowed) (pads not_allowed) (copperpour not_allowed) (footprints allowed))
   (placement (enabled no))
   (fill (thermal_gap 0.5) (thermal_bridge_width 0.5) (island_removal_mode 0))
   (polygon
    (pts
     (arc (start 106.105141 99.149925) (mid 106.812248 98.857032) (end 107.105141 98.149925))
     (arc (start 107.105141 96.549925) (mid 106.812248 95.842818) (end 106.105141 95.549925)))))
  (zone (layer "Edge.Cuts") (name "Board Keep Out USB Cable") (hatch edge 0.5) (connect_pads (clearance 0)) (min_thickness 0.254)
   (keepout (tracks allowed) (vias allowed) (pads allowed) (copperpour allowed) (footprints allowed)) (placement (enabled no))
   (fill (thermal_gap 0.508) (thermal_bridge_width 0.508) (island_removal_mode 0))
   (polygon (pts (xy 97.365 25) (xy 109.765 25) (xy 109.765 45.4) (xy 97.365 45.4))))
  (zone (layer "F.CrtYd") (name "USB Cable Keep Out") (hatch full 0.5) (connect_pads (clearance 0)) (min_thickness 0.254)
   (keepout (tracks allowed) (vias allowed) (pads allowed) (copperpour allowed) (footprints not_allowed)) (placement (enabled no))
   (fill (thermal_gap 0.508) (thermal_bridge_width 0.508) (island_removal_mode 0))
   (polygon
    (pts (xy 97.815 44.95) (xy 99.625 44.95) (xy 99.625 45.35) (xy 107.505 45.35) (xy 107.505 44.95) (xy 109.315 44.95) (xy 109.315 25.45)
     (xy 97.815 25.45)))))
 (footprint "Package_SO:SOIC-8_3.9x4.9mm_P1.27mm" (layer "F.Cu") (at 119.855 57.85)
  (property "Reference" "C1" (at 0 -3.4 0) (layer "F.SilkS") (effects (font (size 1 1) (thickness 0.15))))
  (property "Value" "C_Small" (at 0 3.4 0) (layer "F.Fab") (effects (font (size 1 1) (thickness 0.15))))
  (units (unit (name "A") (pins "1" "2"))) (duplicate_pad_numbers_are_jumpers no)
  (pad "1" smd roundrect (at -2.475 -1.905) (size 1.95 0.6) (layers "F.Cu" "F.Mask" "F.Paste") (roundrect_rratio 0.25) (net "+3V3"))
  (pad "2" smd roundrect (at -2.475 -0.635) (size 1.95 0.6) (layers "F.Cu" "F.Mask" "F.Paste") (roundrect_rratio 0.25) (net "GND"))
  (pad "3" smd roundrect (at -2.475 0.635) (size 1.95 0.6) (layers "F.Cu" "F.Mask" "F.Paste") (roundrect_rratio 0.25))
  (pad "4" smd roundrect (at -2.475 1.905) (size 1.95 0.6) (layers "F.Cu" "F.Mask" "F.Paste") (roundrect_rratio 0.25))
  (pad "5" smd roundrect (at 2.475 1.905) (size 1.95 0.6) (layers "F.Cu" "F.Mask" "F.Paste") (roundrect_rratio 0.25))
  (pad "6" smd roundrect (at 2.475 0.635) (size 1.95 0.6) (layers "F.Cu" "F.Mask" "F.Paste") (roundrect_rratio 0.25))
  (pad "7" smd roundrect (at 2.475 -0.635) (size 1.95 0.6) (layers "F.Cu" "F.Mask" "F.Paste") (roundrect_rratio 0.25))
  (pad "8" smd roundrect (at 2.475 -1.905) (size 1.95 0.6) (layers "F.Cu" "F.Mask" "F.Paste") (roundrect_rratio 0.25)))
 (gr_rect (start 80.9746 22.9746) (end 81 23) (stroke (width 0.05) (type default)) (fill no) (layer "Edge.Cuts"))
 (gr_rect (start 89 23.5) (end 134 103.5) (stroke (width 0.05) (type default)) (fill no) (layer "Edge.Cuts"))
 (segment (start 120.475 77.895) (end 121.5 78.92) (width 0.2) (layer "F.Cu") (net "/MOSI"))
 (segment (start 111.35 78.19082) (end 111.64582 77.895) (width 0.2) (layer "F.Cu") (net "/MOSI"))
 (segment (start 111.64582 77.895) (end 120.475 77.895) (width 0.2) (layer "F.Cu") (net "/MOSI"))
 (segment (start 113.255 86.62) (end 111.35 84.715) (width 0.2) (layer "F.Cu") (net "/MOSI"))
 (segment (start 111.35 84.715) (end 111.35 78.19082) (width 0.2) (layer "F.Cu") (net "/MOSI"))
 (segment (start 113.255 48.52) (end 113.255 51.06) (width 0.2) (layer "F.Cu") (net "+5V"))
 (segment (start 122.216346 87.69) (end 116.865 87.69) (width 0.2) (layer "F.Cu") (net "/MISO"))
 (segment (start 121.5 81.46) (end 122.65 82.61) (width 0.2) (layer "F.Cu") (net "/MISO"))
 (segment (start 122.65 87.256346) (end 122.216346 87.69) (width 0.2) (layer "F.Cu") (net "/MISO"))
 (segment (start 116.865 87.69) (end 113.255 84.08) (width 0.2) (layer "F.Cu") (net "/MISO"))
 (segment (start 122.65 82.61) (end 122.65 87.256346) (width 0.2) (layer "F.Cu") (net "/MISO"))
 (segment (start 113.255 53.6) (end 116.87 57.215) (width 0.2) (layer "F.Cu") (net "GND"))
 (segment (start 114.510636 62.66) (end 120.35 68.499364) (width 0.2) (layer "F.Cu") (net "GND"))
 (segment (start 120.35 68.499364) (end 120.35 72.69) (width 0.2) (layer "F.Cu") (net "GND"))
 (segment (start 95.775 67.4) (end 94.675 66.3) (width 0.2) (layer "F.Cu") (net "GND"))
 (segment (start 94.675 79) (end 95.775 77.9) (width 0.2) (layer "F.Cu") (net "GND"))
 (segment (start 94.675 91.7) (end 95.775 90.6) (width 0.2) (layer "F.Cu") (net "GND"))
 (segment (start 110.255 53.6) (end 111.355 54.7) (width 0.2) (layer "F.Cu") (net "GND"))
 (segment (start 113.96 79) (end 113.255 79) (width 0.2) (layer "F.Cu") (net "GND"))
 (segment (start 113.070636 53.6) (end 112.455 53.6) (width 0.2) (layer "F.Cu") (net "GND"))
 (segment (start 94.675 66.3) (end 94.059364 66.3) (width 0.2) (layer "F.Cu") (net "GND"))
 (segment (start 117.38 57.215) (end 116.685636 57.215) (width 0.2) (layer "F.Cu") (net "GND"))
 (segment (start 111.355 61.675636) (end 112.339364 62.66) (width 0.2) (layer "F.Cu") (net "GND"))
 (segment (start 91.975 55.5) (end 93.875 53.6) (width 0.2) (layer "F.Cu") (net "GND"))
 (segment (start 94.675 53.6) (end 110.255 53.6) (width 0.2) (layer "F.Cu") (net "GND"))
 (segment (start 112.339364 62.66) (end 114.510636 62.66) (width 0.2) (layer "F.Cu") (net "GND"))
 (segment (start 121.5 86.54) (end 113.96 79) (width 0.2) (layer "F.Cu") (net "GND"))
 (segment (start 120.35 72.69) (end 121.5 73.84) (width 0.2) (layer "F.Cu") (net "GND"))
 (segment (start 91.975 64.215636) (end 91.975 55.5) (width 0.2) (layer "F.Cu") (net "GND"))
 (segment (start 95.775 90.6) (end 95.775 80.1) (width 0.2) (layer "F.Cu") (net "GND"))
 (segment (start 95.775 77.9) (end 95.775 67.4) (width 0.2) (layer "F.Cu") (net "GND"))
 (segment (start 95.775 80.1) (end 94.675 79) (width 0.2) (layer "F.Cu") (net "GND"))
 (segment (start 112.455 53.6) (end 111.355 54.7) (width 0.2) (layer "F.Cu") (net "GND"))
 (segment (start 116.685636 57.215) (end 113.070636 53.6) (width 0.2) (layer "F.Cu") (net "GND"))
 (segment (start 116.87 57.215) (end 117.38 57.215) (width 0.2) (layer "F.Cu") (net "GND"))
 (segment (start 111.355 54.7) (end 111.355 61.675636) (width 0.2) (layer "F.Cu") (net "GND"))
 (segment (start 94.059364 66.3) (end 91.975 64.215636) (width 0.2) (layer "F.Cu") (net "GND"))
 (segment (start 121.5 86.54) (end 116.34 91.7) (width 0.2) (layer "B.Cu") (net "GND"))
 (segment (start 116.34 91.7) (end 112.455 91.7) (width 0.2) (layer "B.Cu") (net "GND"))
 (segment (start 117.615 73.84) (end 121.5 73.84) (width 0.2) (layer "B.Cu") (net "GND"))
 (segment (start 112.455 79) (end 117.615 73.84) (width 0.2) (layer "B.Cu") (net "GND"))
 (segment (start 115.84 89.16) (end 112.455 89.16) (width 0.2) (layer "B.Cu") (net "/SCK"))
 (segment (start 121 84) (end 115.84 89.16) (width 0.2) (layer "B.Cu") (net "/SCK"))
 (segment (start 121.5 84) (end 121 84) (width 0.2) (layer "B.Cu") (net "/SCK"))
 (segment (start 121.023654 74.99) (end 115.16 69.126346) (width 0.2) (layer "F.Cu") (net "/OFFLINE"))
 (segment (start 101.360504 62.7) (end 100.250635 62.7) (width 0.2) (layer "F.Cu") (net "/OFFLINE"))
 (segment (start 114.512708 67.405) (end 106.065504 67.405) (width 0.2) (layer "F.Cu") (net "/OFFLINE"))
 (segment (start 93.875 56.324365) (end 93.875 56.14) (width 0.2) (layer "F.Cu") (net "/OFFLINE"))
 (segment (start 100.250635 62.7) (end 93.875 56.324365) (width 0.2) (layer "F.Cu") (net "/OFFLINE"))
 (segment (start 106.065504 67.405) (end 101.360504 62.7) (width 0.2) (layer "F.Cu") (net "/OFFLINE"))
 (segment (start 115.16 69.126346) (end 115.16 68.052292) (width 0.2) (layer "F.Cu") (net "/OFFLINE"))
 (segment (start 122.65 74.316346) (end 121.976346 74.99) (width 0.2) (layer "F.Cu") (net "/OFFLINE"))
 (segment (start 121.5 68.76) (end 122.65 69.91) (width 0.2) (layer "F.Cu") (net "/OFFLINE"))
 (segment (start 122.65 69.91) (end 122.65 74.316346) (width 0.2) (layer "F.Cu") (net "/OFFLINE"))
 (segment (start 115.16 68.052292) (end 114.512708 67.405) (width 0.2) (layer "F.Cu") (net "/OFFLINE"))
 (segment (start 121.976346 74.99) (end 121.023654 74.99) (width 0.2) (layer "F.Cu") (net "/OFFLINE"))
 (segment (start 93.54363 51.06) (end 91.575 53.02863) (width 0.2) (layer "F.Cu") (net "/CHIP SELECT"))
 (segment (start 110.95 76.409365) (end 111.999365 75.36) (width 0.2) (layer "F.Cu") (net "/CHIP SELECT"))
 (segment (start 93.989364 99.25) (end 107.445 99.25) (width 0.2) (layer "F.Cu") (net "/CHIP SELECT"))
 (segment (start 111.655 94.24) (end 110.95 93.535) (width 0.2) (layer "F.Cu") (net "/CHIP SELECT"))
 (segment (start 120.48 75.36) (end 121.5 76.38) (width 0.2) (layer "F.Cu") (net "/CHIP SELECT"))
 (segment (start 107.445 99.25) (end 112.455 94.24) (width 0.2) (layer "F.Cu") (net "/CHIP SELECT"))
 (segment (start 110.95 93.535) (end 110.95 76.409365) (width 0.2) (layer "F.Cu") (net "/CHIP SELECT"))
 (segment (start 111.999365 75.36) (end 120.48 75.36) (width 0.2) (layer "F.Cu") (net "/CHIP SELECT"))
 (segment (start 91.575 53.02863) (end 91.575 96.835636) (width 0.2) (layer "F.Cu") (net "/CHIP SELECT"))
 (segment (start 94.675 51.06) (end 93.54363 51.06) (width 0.2) (layer "F.Cu") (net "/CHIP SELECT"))
 (segment (start 113.255 94.24) (end 111.655 94.24) (width 0.2) (layer "F.Cu") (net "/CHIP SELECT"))
 (segment (start 91.575 96.835636) (end 93.989364 99.25) (width 0.2) (layer "F.Cu") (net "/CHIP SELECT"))
 (segment (start 120.14 69.94) (end 105.935 69.94) (width 0.2) (layer "B.Cu") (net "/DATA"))
 (segment (start 121.5 71.3) (end 120.14 69.94) (width 0.2) (layer "B.Cu") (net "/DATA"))
 (segment (start 105.935 69.94) (end 94.675 58.68) (width 0.2) (layer "B.Cu") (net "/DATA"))
 (segment (start 123.05 87.53) (end 121.5 89.08) (width 0.2) (layer "F.Cu") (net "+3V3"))
 (segment (start 118.655 57.555552) (end 118.655 56.245001) (width 0.2) (layer "F.Cu") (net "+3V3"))
 (segment (start 118.395552 57.815) (end 118.655 57.555552) (width 0.2) (layer "F.Cu") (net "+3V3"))
 (segment (start 123.05 68.683654) (end 123.05 87.53) (width 0.2) (layer "F.Cu") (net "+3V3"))
 (segment (start 120.35 67.37) (end 121.736346 67.37) (width 0.2) (layer "F.Cu") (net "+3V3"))
 (segment (start 113.255 58.68) (end 114.12 57.815) (width 0.2) (layer "F.Cu") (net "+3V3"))
 (segment (start 118.655 56.245001) (end 118.354999 55.945) (width 0.2) (layer "F.Cu") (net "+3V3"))
 (segment (start 121.736346 67.37) (end 123.05 68.683654) (width 0.2) (layer "F.Cu") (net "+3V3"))
 (segment (start 118.655 65.675) (end 120.35 67.37) (width 0.2) (layer "F.Cu") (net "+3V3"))
 (segment (start 114.12 57.815) (end 118.395552 57.815) (width 0.2) (layer "F.Cu") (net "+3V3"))
 (segment (start 121.5 91.62) (end 121.5 89.08) (width 0.2) (layer "F.Cu") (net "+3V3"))
 (segment (start 118.655 57.555552) (end 118.655 65.675) (width 0.2) (layer "F.Cu") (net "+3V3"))
 (segment (start 118.354999 55.945) (end 117.38 55.945) (width 0.2) (layer "F.Cu") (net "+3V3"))
 (segment (start 111.14082 53) (end 111.64582 52.495) (width 0.2) (layer "F.Cu") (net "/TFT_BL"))
 (segment (start 121.023654 65.743654) (end 121.5 66.22) (width 0.2) (layer "F.Cu") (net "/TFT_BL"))
 (segment (start 111.64582 52.495) (end 115.545552 52.495) (width 0.2) (layer "F.Cu") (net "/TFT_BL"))
 (segment (start 115.545552 52.495) (end 121.023654 57.973102) (width 0.2) (layer "F.Cu") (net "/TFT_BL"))
 (segment (start 98.355 53) (end 111.14082 53) (width 0.2) (layer "F.Cu") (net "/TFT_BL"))
 (segment (start 93.875 48.52) (end 98.355 53) (width 0.2) (layer "F.Cu") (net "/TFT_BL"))
 (segment (start 121.023654 57.973102) (end 121.023654 65.743654) (width 0.2) (layer "F.Cu") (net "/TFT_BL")))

